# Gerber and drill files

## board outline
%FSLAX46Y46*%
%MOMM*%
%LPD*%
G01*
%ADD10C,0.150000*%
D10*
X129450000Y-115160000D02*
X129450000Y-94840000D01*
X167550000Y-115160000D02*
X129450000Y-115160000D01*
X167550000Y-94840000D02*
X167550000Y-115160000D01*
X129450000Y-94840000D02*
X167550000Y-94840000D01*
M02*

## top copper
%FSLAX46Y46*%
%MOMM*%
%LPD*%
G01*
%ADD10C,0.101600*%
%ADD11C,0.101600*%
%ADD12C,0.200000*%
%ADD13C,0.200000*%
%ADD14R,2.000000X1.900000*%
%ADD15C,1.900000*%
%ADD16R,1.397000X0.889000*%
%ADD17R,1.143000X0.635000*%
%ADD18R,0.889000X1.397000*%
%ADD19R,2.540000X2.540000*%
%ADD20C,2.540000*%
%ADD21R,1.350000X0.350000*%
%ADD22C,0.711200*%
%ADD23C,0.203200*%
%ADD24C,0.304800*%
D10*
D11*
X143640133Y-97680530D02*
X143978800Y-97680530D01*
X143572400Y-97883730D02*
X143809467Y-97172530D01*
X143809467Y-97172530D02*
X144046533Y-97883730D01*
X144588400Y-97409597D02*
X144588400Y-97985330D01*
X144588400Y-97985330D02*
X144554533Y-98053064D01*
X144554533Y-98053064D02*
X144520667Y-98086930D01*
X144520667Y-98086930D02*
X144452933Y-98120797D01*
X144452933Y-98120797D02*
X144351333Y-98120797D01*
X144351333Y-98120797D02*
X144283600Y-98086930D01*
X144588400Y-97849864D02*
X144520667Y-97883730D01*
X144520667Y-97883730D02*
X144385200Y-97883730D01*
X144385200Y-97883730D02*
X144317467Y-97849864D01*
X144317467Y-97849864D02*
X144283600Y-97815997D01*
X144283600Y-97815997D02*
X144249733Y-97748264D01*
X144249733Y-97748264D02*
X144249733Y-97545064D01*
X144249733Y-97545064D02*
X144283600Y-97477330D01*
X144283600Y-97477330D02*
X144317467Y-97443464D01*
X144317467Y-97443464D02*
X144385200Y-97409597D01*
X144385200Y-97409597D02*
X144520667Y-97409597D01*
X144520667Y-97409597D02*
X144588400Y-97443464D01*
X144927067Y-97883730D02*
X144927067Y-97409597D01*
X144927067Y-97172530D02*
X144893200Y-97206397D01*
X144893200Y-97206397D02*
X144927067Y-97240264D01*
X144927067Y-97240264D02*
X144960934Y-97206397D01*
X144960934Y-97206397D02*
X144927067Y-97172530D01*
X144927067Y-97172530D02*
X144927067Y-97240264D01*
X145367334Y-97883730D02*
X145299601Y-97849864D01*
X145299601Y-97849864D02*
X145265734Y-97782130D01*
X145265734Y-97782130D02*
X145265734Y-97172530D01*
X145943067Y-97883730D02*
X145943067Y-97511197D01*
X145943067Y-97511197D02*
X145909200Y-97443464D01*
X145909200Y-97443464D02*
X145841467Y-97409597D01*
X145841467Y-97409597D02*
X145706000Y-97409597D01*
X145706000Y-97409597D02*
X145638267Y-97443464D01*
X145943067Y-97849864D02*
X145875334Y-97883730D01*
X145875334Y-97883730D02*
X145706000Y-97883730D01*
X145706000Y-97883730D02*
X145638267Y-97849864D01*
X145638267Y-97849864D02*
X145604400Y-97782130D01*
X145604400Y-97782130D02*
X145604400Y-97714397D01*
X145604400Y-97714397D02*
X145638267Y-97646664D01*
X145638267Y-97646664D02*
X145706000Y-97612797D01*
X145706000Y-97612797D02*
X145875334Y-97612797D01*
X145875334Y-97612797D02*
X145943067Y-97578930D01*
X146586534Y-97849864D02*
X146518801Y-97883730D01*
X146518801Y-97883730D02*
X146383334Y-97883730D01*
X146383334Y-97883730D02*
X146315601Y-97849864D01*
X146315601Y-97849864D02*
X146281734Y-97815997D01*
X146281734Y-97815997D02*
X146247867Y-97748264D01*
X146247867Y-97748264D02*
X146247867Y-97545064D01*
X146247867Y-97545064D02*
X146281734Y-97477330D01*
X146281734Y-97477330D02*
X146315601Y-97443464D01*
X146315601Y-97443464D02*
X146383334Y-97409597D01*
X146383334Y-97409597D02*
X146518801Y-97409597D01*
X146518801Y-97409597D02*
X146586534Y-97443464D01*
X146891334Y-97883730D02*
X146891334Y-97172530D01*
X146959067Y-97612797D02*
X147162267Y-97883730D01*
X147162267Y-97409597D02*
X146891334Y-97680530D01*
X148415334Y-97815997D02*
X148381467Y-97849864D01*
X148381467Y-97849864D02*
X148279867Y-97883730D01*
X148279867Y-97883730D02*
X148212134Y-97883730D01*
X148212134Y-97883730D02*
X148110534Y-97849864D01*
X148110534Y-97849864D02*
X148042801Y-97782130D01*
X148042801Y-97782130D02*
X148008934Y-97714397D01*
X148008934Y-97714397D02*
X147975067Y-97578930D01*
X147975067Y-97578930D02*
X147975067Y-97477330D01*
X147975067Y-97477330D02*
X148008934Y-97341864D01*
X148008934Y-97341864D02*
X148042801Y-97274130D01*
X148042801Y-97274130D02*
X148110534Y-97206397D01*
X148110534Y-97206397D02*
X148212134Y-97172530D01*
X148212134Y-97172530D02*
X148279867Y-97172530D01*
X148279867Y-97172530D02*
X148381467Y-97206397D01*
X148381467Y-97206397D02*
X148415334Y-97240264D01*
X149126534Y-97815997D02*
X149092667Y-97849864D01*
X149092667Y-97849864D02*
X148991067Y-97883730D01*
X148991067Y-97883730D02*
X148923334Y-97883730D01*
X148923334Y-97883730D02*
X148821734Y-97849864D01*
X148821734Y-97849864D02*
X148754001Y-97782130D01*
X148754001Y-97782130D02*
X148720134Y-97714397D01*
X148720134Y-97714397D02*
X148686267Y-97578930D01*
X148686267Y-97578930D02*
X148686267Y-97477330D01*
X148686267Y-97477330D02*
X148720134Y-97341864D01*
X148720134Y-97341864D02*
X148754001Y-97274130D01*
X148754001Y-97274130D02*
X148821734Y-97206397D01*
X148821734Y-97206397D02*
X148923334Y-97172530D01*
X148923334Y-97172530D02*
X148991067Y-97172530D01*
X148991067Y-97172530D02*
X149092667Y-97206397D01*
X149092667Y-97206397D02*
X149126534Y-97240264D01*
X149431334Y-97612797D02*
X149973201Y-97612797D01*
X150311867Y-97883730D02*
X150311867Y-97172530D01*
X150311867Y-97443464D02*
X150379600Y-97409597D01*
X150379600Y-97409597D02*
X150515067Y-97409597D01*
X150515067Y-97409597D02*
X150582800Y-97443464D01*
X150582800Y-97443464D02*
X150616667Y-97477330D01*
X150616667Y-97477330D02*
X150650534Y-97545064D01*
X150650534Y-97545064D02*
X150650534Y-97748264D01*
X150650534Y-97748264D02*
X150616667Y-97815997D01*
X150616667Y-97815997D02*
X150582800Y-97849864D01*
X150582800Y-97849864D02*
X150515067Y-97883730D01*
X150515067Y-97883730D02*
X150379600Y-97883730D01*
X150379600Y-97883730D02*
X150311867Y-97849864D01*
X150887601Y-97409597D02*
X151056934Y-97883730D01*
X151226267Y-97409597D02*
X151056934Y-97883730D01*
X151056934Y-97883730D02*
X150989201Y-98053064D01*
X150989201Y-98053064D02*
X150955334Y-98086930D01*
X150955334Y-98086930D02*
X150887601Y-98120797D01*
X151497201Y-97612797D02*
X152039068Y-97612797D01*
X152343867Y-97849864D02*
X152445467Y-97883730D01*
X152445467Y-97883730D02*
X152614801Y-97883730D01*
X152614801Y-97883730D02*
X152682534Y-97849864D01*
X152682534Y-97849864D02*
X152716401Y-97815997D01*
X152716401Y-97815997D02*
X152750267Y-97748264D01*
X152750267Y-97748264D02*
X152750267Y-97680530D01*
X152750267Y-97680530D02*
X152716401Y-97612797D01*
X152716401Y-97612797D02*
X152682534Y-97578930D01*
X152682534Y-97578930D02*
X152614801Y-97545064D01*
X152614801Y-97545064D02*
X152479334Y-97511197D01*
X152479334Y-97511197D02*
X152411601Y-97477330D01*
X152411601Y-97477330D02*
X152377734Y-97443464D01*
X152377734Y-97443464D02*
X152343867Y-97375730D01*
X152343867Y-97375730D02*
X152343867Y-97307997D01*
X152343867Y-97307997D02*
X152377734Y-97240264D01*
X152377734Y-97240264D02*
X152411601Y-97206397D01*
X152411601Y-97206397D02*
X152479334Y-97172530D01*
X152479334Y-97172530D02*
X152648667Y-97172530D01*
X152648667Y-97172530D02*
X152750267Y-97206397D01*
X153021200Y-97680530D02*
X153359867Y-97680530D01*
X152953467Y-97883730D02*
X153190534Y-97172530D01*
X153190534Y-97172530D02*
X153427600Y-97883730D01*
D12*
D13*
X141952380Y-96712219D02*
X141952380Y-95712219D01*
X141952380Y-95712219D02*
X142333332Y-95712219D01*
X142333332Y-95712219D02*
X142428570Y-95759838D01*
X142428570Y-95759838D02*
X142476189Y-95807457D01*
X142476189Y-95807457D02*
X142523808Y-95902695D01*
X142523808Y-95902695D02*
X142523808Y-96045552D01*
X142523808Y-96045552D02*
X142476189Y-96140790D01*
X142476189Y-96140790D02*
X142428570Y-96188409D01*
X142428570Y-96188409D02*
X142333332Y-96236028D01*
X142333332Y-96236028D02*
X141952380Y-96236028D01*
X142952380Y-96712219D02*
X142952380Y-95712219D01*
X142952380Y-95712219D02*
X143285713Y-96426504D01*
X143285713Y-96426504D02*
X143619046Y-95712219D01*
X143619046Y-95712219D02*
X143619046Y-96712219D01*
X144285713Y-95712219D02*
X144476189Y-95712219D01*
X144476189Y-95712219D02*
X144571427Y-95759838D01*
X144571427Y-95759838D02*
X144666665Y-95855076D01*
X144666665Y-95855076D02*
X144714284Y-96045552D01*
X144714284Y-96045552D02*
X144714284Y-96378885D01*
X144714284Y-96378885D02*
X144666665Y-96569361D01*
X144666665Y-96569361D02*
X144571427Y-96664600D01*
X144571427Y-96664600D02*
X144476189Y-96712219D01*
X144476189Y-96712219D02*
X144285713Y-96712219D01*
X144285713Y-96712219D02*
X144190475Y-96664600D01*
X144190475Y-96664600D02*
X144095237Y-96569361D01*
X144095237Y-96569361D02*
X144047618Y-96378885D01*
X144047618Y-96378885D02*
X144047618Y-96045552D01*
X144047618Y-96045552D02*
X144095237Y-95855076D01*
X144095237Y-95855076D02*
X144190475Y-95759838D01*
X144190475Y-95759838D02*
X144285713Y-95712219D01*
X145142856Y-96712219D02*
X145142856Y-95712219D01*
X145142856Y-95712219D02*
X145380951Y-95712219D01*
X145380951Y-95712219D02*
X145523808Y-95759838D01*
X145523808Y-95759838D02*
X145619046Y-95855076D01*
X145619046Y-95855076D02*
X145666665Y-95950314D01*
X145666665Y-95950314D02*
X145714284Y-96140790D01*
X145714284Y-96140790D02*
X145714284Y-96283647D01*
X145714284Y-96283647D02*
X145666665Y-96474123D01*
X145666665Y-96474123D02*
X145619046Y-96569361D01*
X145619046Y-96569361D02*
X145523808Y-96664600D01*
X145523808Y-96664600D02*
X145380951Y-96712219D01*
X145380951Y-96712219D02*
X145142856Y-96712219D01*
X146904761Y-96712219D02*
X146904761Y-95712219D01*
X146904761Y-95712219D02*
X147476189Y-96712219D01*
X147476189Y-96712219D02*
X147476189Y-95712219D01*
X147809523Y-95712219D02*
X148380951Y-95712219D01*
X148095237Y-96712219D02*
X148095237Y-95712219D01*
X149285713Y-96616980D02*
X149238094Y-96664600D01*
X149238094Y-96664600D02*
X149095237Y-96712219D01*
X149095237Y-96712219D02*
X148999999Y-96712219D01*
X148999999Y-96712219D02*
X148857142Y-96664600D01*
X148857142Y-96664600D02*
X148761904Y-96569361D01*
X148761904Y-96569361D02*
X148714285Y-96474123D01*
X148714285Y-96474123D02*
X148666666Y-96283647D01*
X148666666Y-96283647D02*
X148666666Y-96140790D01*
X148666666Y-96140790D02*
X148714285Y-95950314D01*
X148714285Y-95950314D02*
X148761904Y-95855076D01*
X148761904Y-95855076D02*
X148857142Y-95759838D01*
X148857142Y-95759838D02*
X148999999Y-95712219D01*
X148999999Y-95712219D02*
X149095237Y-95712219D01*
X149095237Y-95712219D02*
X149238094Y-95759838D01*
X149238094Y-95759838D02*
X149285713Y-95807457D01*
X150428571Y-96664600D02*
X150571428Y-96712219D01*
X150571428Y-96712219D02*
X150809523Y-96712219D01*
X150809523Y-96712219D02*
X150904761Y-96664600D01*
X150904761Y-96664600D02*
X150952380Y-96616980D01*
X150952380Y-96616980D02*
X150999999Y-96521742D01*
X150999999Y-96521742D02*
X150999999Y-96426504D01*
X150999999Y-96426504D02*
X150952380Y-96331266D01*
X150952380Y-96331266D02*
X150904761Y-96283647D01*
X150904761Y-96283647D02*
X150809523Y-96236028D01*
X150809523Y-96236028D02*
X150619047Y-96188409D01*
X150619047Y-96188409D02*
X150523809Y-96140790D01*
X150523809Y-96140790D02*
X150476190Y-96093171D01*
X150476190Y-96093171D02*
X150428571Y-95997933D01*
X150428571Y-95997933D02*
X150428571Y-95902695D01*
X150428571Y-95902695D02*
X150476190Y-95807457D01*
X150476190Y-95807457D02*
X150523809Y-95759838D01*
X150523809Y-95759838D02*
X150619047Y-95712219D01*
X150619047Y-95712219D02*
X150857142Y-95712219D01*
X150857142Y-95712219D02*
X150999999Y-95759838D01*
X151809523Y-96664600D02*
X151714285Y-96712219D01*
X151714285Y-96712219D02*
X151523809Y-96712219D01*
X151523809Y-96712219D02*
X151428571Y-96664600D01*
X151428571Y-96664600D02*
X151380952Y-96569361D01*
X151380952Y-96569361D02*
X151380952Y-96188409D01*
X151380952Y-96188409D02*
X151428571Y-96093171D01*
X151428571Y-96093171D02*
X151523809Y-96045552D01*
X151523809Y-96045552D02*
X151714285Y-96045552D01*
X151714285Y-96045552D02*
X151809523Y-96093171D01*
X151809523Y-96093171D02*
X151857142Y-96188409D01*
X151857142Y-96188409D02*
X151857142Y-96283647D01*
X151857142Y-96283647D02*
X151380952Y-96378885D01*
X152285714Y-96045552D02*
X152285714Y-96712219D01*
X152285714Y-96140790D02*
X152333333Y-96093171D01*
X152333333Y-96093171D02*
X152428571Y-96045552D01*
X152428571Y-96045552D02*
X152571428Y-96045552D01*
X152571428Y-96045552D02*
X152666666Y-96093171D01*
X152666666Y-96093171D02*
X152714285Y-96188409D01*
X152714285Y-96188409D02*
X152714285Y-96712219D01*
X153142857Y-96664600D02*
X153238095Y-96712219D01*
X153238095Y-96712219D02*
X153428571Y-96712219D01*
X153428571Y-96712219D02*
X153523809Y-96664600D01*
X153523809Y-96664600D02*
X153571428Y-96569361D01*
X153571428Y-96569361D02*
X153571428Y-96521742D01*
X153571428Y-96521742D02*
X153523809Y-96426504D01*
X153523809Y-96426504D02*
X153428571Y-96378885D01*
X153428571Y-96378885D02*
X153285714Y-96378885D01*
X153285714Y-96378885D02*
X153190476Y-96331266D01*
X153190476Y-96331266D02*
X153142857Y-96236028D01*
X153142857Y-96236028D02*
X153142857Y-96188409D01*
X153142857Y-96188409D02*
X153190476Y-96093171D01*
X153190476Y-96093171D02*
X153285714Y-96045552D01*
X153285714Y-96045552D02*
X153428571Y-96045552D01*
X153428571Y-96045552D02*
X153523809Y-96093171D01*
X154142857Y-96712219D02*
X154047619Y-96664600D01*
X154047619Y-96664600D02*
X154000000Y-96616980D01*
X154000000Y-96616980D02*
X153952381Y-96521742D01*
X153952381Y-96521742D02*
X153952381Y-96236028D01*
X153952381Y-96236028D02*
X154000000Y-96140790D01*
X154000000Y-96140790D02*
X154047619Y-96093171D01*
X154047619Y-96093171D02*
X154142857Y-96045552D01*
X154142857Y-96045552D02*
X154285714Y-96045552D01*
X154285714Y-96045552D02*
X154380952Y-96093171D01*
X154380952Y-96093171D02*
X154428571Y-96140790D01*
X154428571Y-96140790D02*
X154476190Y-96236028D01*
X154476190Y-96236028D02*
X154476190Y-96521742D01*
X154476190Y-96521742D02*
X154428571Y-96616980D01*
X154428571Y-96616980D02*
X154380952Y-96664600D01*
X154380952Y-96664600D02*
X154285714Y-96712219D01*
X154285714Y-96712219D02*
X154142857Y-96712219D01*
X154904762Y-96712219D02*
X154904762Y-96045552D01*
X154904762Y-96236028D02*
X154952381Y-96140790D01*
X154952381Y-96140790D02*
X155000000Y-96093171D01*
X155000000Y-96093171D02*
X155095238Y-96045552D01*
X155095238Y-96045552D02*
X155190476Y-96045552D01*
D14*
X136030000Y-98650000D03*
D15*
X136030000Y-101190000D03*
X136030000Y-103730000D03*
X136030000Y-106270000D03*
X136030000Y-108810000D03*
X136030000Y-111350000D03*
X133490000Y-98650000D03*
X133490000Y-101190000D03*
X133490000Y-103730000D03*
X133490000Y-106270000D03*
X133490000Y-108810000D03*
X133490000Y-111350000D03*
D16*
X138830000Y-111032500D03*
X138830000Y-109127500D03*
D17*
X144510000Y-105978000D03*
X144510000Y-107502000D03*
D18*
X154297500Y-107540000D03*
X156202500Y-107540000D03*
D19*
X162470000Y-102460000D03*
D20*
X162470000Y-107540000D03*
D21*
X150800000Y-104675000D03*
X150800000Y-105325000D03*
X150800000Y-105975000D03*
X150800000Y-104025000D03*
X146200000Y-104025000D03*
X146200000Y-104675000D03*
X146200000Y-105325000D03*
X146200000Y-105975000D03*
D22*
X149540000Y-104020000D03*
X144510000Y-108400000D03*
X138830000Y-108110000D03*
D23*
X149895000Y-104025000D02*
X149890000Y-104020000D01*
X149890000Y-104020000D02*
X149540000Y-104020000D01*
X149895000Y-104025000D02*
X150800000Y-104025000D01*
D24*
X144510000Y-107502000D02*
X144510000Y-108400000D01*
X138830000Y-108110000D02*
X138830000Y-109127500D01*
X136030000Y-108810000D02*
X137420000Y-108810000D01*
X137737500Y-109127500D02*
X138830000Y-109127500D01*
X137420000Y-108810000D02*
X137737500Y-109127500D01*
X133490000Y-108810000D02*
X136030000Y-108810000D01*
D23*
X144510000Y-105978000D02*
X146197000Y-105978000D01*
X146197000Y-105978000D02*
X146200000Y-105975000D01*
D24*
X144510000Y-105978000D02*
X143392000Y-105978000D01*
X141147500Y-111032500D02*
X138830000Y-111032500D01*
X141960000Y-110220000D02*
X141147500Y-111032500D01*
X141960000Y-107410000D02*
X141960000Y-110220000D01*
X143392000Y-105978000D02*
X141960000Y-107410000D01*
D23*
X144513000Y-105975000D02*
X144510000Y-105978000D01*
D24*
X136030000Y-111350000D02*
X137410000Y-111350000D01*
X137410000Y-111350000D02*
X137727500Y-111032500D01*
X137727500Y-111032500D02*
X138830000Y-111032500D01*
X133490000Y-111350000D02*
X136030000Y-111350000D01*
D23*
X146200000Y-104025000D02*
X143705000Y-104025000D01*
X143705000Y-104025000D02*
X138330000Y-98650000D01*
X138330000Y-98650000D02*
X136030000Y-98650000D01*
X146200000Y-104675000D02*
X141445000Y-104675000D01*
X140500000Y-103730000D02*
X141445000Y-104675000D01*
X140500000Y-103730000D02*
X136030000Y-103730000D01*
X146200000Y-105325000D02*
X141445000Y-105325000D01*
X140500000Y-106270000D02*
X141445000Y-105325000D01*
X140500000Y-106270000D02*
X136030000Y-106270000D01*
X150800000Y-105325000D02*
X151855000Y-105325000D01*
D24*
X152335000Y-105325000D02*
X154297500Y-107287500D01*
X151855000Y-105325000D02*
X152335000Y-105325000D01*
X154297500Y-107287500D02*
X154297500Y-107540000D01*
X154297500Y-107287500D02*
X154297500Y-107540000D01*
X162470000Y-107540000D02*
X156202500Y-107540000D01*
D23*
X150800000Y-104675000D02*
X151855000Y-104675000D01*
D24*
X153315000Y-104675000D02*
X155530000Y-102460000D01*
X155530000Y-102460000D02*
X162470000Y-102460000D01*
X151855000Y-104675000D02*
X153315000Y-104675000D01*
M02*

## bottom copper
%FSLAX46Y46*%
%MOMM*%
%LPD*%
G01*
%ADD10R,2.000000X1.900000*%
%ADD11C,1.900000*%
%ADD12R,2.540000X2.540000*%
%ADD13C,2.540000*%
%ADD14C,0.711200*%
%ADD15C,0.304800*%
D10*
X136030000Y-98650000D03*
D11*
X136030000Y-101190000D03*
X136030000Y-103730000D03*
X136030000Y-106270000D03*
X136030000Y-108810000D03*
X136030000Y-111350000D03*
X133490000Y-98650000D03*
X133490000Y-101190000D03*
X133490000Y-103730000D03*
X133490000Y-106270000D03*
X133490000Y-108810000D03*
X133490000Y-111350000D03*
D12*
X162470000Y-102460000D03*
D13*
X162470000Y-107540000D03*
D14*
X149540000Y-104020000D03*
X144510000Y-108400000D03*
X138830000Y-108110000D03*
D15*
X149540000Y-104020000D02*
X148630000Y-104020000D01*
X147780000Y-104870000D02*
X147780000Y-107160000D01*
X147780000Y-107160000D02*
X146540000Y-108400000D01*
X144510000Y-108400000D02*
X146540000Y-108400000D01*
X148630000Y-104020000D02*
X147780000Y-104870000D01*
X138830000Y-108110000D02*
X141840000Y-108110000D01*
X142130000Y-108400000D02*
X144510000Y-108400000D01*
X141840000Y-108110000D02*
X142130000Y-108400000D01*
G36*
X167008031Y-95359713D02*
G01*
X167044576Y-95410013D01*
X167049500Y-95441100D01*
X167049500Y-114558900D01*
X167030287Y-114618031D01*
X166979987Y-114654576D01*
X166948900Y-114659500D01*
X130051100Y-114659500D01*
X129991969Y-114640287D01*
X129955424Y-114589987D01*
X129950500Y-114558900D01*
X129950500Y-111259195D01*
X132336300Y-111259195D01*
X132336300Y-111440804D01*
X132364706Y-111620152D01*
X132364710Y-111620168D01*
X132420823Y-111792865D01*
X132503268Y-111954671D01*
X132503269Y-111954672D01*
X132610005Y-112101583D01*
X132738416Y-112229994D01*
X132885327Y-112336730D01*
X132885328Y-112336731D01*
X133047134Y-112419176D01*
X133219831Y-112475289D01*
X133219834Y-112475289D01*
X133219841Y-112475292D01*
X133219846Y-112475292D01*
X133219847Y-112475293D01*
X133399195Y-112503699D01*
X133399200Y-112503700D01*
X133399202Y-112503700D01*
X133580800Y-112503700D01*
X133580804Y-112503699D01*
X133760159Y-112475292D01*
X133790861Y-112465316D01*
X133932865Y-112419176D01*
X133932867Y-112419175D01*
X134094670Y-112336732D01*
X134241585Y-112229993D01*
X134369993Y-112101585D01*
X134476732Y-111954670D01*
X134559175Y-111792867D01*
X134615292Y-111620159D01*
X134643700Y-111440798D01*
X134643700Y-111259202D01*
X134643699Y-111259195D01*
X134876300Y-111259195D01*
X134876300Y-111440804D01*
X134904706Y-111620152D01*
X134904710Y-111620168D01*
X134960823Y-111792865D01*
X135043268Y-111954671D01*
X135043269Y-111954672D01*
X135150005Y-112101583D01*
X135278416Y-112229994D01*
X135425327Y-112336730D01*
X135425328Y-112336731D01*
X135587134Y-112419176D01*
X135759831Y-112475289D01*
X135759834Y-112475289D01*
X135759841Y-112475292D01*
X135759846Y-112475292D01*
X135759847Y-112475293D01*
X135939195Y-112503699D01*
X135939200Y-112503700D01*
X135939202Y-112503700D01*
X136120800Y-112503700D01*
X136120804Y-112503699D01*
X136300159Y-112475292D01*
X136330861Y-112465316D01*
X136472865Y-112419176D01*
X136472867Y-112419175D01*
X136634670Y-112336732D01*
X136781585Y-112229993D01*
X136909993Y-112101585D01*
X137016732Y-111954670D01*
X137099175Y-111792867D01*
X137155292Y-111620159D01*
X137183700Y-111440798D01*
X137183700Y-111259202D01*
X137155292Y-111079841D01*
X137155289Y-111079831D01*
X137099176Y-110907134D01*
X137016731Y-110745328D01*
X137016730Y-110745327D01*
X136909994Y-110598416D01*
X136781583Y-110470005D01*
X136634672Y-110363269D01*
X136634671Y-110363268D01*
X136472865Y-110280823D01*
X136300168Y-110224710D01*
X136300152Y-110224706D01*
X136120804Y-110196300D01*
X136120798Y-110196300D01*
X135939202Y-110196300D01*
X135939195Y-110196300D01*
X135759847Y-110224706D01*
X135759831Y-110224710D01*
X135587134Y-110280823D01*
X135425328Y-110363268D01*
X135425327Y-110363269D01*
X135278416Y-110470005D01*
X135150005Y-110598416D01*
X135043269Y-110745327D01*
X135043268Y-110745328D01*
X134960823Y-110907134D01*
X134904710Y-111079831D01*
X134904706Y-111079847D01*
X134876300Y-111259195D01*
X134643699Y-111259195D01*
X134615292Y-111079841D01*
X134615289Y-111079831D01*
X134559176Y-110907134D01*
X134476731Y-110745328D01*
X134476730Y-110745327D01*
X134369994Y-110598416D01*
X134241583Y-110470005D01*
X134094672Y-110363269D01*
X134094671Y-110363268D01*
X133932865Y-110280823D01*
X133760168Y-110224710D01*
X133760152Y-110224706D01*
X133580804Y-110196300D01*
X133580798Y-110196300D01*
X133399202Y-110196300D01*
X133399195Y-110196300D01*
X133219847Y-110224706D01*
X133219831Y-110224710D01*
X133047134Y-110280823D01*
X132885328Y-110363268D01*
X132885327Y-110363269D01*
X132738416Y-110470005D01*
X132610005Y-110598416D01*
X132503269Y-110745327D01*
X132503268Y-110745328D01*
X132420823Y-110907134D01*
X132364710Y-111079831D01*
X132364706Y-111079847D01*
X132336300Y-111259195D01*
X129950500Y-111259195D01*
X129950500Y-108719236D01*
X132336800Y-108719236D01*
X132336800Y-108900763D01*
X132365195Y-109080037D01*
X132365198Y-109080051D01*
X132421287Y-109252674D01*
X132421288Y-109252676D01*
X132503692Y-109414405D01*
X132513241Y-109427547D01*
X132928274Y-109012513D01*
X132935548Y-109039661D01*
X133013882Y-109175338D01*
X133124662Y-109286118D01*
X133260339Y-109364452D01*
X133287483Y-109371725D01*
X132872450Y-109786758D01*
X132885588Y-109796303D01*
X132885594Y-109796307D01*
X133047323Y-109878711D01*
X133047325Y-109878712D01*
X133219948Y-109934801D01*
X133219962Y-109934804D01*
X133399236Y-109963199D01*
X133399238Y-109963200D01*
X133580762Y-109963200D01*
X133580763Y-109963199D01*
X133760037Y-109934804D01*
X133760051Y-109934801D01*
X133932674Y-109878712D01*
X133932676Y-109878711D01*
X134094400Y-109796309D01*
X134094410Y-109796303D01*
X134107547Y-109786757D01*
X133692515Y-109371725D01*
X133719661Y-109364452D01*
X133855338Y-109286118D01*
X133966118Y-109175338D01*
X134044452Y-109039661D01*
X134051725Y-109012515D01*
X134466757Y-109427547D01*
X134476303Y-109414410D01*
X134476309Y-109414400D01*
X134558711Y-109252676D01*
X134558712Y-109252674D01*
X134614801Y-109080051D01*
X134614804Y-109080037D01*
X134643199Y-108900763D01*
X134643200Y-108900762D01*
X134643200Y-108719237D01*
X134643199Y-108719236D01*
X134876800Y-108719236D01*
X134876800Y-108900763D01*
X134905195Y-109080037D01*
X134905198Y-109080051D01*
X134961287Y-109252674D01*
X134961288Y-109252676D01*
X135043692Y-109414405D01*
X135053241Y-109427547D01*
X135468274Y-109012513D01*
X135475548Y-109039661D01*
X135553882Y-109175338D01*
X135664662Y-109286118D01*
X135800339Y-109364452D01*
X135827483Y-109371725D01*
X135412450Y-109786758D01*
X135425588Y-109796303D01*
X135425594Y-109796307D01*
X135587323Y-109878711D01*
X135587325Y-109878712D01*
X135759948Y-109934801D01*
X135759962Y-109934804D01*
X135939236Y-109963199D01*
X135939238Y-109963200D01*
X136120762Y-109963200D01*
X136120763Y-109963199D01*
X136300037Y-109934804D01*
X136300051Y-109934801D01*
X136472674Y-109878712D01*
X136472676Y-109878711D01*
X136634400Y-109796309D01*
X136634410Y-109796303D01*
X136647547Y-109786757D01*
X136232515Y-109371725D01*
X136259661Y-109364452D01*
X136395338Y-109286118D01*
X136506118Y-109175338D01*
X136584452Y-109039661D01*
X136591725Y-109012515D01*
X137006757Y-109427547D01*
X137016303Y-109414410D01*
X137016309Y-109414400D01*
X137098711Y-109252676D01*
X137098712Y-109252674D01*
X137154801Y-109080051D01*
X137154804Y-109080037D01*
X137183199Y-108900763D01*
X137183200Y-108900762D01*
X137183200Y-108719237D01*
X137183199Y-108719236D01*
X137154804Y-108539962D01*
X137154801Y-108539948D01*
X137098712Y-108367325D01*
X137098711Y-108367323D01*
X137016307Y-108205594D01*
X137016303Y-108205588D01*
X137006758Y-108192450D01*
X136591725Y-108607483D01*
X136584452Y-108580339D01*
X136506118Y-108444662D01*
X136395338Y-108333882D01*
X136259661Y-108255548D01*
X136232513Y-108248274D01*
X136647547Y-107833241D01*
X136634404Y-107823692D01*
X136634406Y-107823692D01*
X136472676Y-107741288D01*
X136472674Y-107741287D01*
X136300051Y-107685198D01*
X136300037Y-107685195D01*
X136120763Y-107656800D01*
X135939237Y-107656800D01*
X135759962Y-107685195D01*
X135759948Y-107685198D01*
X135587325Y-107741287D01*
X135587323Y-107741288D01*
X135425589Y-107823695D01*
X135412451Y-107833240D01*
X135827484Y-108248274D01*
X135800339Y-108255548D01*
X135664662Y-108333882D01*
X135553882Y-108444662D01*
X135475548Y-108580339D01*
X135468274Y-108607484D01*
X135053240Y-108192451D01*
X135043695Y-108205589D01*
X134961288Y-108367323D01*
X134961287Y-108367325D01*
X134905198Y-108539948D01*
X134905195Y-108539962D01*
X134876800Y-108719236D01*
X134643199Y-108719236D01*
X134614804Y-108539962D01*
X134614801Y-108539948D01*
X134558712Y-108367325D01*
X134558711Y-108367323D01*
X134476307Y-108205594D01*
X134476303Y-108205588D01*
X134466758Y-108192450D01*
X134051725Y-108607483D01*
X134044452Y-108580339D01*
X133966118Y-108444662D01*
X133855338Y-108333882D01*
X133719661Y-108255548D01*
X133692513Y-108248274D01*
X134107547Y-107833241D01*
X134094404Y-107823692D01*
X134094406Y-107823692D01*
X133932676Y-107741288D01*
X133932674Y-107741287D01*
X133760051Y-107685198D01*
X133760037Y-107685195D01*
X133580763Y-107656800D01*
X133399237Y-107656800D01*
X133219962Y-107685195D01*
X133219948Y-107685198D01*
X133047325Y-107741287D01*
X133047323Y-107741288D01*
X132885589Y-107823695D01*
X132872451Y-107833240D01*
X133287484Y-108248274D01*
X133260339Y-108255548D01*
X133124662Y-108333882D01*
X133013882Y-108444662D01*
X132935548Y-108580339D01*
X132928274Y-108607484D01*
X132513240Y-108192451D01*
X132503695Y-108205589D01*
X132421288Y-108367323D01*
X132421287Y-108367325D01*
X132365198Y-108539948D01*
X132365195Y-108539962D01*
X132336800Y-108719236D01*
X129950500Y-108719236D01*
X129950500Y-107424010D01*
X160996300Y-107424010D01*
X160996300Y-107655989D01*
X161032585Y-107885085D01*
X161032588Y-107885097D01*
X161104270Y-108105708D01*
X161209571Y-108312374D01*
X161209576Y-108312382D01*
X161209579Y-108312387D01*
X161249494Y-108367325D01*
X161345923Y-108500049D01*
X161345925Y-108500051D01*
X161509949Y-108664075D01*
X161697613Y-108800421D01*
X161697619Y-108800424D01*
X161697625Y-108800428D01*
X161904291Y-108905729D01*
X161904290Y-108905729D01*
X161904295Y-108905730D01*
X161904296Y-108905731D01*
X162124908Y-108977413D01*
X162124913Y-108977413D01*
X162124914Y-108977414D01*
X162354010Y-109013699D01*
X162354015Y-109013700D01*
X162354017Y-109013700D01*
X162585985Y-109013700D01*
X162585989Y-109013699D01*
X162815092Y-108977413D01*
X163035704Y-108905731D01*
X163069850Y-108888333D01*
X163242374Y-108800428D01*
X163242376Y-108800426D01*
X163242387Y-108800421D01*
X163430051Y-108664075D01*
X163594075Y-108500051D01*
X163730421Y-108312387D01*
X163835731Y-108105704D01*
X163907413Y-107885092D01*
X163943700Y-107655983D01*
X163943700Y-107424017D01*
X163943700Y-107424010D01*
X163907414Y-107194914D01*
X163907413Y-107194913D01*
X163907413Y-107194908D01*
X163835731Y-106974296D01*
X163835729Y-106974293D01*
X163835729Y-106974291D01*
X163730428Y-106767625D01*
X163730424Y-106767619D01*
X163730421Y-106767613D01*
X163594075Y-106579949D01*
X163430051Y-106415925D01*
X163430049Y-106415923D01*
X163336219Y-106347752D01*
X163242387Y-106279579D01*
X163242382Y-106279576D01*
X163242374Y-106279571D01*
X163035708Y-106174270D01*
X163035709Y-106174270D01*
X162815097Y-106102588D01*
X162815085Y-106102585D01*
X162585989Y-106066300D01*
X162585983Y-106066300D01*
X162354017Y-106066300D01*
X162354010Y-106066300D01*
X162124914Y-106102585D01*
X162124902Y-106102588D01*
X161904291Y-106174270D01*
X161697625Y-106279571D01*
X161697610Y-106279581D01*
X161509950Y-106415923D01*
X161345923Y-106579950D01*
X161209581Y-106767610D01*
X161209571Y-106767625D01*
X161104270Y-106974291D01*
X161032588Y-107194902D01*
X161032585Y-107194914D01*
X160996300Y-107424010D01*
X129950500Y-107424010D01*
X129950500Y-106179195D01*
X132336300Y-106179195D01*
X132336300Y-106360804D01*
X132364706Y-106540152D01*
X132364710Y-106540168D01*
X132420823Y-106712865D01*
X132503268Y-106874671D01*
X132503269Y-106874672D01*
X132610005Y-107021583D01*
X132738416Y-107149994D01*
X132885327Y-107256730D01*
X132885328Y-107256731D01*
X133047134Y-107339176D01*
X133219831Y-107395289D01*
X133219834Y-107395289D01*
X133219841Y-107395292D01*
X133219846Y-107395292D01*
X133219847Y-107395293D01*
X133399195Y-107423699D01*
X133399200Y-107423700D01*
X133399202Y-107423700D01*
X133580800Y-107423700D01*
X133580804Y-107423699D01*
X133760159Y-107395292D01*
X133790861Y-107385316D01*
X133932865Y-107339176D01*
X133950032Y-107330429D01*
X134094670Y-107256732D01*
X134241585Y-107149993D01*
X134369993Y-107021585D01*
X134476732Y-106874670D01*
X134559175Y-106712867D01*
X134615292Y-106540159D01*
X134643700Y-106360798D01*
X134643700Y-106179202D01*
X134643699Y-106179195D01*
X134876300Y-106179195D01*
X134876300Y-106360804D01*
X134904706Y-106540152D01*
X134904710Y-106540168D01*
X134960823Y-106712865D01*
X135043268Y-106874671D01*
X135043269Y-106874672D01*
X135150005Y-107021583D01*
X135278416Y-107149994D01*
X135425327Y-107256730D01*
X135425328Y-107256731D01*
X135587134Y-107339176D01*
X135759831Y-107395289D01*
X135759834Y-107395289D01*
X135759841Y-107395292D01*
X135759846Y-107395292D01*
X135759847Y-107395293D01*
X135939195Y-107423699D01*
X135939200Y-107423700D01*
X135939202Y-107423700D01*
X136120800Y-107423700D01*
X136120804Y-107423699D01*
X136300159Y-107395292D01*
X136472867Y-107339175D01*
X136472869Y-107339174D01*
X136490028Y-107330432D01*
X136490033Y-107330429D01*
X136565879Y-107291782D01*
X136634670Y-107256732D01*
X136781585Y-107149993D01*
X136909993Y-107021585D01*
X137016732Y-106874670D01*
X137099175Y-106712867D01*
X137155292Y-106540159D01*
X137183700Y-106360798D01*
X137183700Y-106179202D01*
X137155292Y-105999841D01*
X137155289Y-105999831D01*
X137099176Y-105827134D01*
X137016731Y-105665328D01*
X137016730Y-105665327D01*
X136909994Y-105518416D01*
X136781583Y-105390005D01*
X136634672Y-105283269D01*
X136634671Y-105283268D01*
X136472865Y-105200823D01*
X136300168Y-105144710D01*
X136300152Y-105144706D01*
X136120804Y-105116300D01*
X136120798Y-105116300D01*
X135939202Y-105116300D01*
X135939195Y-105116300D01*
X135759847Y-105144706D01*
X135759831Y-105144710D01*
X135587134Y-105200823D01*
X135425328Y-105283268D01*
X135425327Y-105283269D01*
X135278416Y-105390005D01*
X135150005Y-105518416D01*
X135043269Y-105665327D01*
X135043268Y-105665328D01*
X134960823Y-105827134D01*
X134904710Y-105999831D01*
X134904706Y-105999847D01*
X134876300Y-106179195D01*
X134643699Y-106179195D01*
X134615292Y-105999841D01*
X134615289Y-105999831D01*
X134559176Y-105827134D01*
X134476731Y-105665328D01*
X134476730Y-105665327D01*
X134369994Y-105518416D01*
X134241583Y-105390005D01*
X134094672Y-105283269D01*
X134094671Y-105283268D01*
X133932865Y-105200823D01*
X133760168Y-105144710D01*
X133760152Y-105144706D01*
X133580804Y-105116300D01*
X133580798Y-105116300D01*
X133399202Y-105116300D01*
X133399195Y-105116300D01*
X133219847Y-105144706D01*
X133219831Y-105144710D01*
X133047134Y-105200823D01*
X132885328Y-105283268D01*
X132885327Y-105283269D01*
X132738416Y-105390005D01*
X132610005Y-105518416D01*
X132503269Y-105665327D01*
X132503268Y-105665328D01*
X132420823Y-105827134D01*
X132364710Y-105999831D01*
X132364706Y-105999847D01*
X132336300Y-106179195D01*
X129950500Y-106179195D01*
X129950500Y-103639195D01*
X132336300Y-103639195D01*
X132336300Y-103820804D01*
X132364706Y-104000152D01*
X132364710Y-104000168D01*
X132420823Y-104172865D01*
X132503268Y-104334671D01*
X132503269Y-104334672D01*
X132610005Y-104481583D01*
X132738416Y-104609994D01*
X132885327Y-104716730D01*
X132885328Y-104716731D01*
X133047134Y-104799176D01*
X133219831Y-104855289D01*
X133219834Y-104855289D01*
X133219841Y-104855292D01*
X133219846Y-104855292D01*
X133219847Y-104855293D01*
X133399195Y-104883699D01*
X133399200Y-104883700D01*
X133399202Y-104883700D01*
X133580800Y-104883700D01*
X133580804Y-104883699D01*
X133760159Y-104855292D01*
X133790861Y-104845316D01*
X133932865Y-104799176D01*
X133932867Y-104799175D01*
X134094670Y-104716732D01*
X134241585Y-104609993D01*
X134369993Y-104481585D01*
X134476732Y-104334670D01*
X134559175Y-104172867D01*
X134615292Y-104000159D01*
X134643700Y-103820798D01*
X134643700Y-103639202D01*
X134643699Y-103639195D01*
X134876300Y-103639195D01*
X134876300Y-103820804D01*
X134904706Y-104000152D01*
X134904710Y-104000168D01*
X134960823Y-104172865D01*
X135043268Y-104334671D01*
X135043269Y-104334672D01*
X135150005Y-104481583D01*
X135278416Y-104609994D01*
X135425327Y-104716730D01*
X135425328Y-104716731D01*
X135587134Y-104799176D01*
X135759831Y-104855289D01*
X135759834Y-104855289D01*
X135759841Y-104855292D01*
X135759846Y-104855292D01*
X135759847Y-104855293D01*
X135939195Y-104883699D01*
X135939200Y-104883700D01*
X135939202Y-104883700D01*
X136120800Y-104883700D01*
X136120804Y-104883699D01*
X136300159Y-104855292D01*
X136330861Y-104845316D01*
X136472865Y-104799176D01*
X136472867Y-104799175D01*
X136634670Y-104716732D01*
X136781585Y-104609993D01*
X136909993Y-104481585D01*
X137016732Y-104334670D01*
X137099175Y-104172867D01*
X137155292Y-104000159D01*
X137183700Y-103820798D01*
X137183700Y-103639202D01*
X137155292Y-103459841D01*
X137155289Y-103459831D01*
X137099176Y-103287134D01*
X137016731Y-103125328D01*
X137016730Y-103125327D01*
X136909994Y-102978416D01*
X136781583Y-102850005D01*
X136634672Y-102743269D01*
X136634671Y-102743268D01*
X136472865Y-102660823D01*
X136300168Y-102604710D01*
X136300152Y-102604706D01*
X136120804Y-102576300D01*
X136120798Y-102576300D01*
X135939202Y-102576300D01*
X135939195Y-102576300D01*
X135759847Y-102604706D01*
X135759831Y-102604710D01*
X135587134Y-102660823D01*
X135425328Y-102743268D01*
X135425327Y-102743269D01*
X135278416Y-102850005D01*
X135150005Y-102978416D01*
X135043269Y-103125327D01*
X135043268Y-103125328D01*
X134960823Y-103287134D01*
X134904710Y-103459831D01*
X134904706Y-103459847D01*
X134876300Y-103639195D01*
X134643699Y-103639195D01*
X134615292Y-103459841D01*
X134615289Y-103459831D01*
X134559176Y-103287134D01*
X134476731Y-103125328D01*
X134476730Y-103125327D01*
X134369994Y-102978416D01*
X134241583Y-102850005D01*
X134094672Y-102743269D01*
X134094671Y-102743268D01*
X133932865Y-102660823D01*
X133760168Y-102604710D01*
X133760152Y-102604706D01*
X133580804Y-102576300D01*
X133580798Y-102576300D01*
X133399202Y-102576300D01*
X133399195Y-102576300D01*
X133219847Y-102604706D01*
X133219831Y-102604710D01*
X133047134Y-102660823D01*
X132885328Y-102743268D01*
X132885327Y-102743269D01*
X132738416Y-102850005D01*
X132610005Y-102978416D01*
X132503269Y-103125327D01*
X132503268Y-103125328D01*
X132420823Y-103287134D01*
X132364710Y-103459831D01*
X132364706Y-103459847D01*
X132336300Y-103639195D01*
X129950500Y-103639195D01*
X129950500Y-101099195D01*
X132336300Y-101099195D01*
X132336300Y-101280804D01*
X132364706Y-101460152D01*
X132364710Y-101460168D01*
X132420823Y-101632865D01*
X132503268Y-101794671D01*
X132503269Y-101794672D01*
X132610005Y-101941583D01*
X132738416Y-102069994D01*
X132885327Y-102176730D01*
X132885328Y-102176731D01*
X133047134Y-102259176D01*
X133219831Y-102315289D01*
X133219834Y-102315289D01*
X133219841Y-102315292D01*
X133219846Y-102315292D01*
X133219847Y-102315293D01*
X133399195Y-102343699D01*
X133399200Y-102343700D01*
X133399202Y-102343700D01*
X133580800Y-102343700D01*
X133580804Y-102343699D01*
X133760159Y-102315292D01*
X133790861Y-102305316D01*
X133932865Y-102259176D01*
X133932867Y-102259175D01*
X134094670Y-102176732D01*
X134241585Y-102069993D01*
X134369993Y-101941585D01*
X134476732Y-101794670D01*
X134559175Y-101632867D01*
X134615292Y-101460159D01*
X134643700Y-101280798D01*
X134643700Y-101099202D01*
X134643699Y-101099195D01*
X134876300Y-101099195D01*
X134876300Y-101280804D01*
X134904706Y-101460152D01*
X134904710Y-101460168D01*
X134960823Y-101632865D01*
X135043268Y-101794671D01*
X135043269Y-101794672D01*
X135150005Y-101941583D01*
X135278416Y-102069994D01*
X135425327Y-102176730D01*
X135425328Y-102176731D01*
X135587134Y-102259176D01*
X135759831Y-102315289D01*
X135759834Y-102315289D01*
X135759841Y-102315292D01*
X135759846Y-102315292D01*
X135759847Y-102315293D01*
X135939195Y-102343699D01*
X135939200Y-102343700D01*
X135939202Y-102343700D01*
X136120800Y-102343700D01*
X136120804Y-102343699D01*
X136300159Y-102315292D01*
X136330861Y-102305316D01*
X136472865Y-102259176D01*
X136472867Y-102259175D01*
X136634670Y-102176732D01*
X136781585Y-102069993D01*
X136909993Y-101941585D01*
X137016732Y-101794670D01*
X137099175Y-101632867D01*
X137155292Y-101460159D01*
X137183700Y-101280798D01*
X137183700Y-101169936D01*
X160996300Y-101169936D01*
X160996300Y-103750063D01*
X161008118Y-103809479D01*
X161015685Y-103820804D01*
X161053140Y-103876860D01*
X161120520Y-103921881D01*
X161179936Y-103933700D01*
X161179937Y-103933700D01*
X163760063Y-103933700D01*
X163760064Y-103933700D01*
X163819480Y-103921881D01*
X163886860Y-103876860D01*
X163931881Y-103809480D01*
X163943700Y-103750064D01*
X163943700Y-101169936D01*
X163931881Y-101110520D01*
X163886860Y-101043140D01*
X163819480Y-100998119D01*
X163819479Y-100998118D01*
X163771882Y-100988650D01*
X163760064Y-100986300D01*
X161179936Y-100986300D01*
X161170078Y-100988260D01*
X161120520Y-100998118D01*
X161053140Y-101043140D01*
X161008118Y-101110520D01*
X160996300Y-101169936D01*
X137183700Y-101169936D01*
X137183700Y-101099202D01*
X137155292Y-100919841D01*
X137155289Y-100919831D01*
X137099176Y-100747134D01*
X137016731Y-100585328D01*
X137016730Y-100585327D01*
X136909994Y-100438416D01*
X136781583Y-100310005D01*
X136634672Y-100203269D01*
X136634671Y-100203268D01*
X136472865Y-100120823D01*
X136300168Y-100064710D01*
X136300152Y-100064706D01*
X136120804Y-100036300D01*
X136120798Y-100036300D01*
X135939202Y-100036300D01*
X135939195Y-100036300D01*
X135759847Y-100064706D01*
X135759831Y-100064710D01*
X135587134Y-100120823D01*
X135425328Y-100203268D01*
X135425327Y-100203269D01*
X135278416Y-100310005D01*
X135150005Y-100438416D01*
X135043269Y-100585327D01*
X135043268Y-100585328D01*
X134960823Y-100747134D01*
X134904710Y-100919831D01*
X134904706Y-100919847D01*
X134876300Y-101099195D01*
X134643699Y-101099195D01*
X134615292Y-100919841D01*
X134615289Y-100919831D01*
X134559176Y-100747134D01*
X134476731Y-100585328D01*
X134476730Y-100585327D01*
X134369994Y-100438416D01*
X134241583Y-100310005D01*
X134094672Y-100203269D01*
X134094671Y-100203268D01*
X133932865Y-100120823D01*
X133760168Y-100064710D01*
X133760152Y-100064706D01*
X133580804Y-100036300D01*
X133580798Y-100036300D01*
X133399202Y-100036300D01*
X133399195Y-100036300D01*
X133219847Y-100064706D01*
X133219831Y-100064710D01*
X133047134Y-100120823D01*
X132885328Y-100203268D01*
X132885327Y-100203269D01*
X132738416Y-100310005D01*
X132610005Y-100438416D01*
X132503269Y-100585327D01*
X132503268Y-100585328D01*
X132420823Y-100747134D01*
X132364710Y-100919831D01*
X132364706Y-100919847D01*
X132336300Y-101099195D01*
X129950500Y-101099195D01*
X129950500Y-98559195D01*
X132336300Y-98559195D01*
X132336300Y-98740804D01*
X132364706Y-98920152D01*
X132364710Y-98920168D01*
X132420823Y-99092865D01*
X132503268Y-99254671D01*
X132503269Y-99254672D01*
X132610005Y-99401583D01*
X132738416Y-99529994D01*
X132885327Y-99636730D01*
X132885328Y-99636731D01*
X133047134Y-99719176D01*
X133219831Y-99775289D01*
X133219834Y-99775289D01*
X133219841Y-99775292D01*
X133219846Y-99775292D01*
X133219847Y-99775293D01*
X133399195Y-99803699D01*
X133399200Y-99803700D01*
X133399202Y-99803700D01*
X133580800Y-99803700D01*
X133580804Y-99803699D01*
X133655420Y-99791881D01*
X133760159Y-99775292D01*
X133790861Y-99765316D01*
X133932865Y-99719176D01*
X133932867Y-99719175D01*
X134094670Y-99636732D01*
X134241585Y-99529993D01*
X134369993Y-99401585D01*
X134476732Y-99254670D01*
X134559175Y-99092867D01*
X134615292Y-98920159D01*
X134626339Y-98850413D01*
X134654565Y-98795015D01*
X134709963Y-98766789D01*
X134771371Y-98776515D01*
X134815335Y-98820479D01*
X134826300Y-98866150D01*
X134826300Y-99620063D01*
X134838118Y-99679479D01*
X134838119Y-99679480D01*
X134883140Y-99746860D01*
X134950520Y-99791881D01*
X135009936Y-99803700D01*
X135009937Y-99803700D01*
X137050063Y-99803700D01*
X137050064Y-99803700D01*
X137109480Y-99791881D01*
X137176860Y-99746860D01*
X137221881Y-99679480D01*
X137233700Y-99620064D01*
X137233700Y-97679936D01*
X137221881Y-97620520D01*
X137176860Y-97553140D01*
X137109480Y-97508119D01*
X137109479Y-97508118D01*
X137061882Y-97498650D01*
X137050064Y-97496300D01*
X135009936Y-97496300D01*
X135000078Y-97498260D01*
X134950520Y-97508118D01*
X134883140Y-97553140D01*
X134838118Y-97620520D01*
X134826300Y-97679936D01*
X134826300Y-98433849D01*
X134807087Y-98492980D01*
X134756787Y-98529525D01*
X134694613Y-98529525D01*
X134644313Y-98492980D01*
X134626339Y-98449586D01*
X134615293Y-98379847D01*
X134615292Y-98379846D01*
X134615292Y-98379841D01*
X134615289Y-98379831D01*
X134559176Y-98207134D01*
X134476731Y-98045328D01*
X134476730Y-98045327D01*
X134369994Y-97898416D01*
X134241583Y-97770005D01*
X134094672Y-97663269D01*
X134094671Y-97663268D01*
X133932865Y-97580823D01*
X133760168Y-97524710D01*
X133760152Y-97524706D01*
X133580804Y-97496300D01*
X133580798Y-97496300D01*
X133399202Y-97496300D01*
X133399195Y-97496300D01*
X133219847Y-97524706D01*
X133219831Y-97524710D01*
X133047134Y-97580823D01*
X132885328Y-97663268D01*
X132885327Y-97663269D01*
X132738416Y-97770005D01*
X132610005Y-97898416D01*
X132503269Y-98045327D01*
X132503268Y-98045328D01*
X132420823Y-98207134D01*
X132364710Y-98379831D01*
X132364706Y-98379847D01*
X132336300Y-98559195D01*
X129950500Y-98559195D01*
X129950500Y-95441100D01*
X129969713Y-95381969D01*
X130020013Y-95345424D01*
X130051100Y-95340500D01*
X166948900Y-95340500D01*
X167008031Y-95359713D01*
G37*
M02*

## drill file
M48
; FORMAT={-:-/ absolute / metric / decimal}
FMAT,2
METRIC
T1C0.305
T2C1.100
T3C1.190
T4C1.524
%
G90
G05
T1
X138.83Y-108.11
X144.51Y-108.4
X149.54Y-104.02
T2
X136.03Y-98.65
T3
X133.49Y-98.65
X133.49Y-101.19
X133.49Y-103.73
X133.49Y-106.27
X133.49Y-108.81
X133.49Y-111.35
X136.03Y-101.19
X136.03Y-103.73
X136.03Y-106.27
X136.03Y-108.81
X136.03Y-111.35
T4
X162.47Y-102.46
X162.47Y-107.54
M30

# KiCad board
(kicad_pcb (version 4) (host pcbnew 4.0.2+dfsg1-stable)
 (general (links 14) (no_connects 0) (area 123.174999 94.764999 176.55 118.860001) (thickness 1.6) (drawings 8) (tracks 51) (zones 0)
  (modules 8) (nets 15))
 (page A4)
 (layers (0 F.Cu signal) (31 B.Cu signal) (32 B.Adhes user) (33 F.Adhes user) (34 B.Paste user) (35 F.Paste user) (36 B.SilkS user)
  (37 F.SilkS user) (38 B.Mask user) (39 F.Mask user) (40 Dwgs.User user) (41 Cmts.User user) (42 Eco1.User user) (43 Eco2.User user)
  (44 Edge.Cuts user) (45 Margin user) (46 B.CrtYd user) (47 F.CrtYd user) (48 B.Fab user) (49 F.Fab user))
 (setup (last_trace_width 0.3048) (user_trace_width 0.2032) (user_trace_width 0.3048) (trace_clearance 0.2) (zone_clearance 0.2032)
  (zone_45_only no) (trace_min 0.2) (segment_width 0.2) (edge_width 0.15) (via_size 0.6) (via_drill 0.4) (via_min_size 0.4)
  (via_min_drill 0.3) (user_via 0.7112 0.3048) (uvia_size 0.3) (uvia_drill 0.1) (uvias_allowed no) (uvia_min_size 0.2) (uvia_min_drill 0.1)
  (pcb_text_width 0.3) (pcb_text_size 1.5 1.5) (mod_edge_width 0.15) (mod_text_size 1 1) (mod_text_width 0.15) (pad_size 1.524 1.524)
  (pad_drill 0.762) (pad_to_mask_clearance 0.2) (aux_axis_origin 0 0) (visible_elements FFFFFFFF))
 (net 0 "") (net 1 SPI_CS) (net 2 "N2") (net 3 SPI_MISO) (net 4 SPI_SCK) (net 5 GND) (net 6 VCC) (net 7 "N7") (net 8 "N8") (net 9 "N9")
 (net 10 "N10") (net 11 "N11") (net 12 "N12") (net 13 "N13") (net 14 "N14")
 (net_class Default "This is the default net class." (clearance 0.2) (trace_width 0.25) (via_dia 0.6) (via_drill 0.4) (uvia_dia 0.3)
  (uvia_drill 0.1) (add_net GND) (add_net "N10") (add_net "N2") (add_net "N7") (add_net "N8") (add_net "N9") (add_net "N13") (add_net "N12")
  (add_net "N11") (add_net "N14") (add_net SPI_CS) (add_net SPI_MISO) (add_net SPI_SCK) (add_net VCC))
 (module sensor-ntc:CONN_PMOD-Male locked (layer F.Cu) (at 133.49 105 90)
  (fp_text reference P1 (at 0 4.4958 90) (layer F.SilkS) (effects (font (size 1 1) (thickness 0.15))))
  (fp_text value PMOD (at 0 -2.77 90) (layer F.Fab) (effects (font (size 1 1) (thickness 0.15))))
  (pad 1 thru_hole rect (at 6.35 2.54 90) (size 1.9 2) (drill 1.1) (layers *.Cu *.Mask) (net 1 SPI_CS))
  (pad 2 thru_hole circle (at 3.81 2.54 90) (size 1.9 1.9) (drill 1.19) (layers *.Cu *.Mask) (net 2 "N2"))
  (pad 3 thru_hole circle (at 1.27 2.54 90) (size 1.9 1.9) (drill 1.19) (layers *.Cu *.Mask) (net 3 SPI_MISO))
  (pad 4 thru_hole circle (at -1.27 2.54 90) (size 1.9 1.9) (drill 1.19) (layers *.Cu *.Mask) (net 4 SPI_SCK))
  (pad 5 thru_hole circle (at -3.81 2.54 90) (size 1.9 1.9) (drill 1.19) (layers *.Cu *.Mask) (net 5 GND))
  (pad 6 thru_hole circle (at -6.35 2.54 90) (size 1.9 1.9) (drill 1.19) (layers *.Cu *.Mask) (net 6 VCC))
  (pad 7 thru_hole circle (at 6.35 0 90) (size 1.9 1.9) (drill 1.19) (layers *.Cu *.Mask) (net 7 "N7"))
  (pad 8 thru_hole circle (at 3.81 0 90) (size 1.9 1.9) (drill 1.19) (layers *.Cu *.Mask) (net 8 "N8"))
  (pad 9 thru_hole circle (at 1.27 0 90) (size 1.9 1.9) (drill 1.19) (layers *.Cu *.Mask) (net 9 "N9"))
  (pad 10 thru_hole circle (at -1.27 0 90) (size 1.9 1.9) (drill 1.19) (layers *.Cu *.Mask) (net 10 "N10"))
  (pad 11 thru_hole circle (at -3.81 0 90) (size 1.9 1.9) (drill 1.19) (layers *.Cu *.Mask) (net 5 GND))
  (pad 12 thru_hole circle (at -6.35 0 90) (size 1.9 1.9) (drill 1.19) (layers *.Cu *.Mask) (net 6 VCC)))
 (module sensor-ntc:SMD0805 (layer F.Cu) (at 138.83 110.08 90)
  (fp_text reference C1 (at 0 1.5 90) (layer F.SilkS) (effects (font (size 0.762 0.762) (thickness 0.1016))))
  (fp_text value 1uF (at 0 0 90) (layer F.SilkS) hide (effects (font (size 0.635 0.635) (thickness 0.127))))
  (pad 1 smd rect (at -0.9525 0 90) (size 0.889 1.397) (layers F.Cu F.Paste F.Mask) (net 6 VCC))
  (pad 2 smd rect (at 0.9525 0 90) (size 0.889 1.397) (layers F.Cu F.Paste F.Mask) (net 5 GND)))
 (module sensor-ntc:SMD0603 (layer F.Cu) (at 144.51 106.74 270)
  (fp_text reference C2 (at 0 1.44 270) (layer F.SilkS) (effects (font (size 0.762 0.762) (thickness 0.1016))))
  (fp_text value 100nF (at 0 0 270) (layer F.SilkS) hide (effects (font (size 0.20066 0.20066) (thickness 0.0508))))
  (pad 1 smd rect (at -0.762 0 270) (size 0.635 1.143) (layers F.Cu F.Paste F.Mask) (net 6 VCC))
  (pad 2 smd rect (at 0.762 0 270) (size 0.635 1.143) (layers F.Cu F.Paste F.Mask) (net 5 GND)))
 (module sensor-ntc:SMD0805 (layer F.Cu) (at 155.25 107.54)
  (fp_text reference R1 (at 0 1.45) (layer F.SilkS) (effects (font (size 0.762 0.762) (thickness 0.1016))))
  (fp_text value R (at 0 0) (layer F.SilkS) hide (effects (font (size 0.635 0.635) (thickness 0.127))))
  (pad 1 smd rect (at -0.9525 0) (size 0.889 1.397) (layers F.Cu F.Paste F.Mask) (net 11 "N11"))
  (pad 2 smd rect (at 0.9525 0) (size 0.889 1.397) (layers F.Cu F.Paste F.Mask) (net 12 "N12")))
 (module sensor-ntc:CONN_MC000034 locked (layer F.Cu) (at 162.47 105 270)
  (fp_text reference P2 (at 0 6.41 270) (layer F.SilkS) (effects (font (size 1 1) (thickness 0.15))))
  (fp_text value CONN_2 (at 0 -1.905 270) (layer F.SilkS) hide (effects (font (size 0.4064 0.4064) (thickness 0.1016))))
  (pad 1 thru_hole rect (at -2.54 0 270) (size 2.54 2.54) (drill 1.524) (layers *.Cu *.Mask F.SilkS) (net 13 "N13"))
  (pad 2 thru_hole circle (at 2.54 0 270) (size 2.54 2.54) (drill 1.524) (layers *.Cu *.Mask F.SilkS) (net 12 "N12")))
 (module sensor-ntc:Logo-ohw (layer F.Cu) (at 148.5 110)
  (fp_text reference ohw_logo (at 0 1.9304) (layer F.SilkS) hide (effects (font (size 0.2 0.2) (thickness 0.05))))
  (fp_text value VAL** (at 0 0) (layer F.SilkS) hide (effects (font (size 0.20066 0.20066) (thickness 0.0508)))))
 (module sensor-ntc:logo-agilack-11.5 (layer F.Cu) (at 161.56 112.74)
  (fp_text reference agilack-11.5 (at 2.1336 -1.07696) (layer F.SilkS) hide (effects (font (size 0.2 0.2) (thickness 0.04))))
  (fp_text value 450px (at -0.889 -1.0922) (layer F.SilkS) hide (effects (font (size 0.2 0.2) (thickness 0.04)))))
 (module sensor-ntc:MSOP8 (layer F.Cu) (at 148.5 105 90)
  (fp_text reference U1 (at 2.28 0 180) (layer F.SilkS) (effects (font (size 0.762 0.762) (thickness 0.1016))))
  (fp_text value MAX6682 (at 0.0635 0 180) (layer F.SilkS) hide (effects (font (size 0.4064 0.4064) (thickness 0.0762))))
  (pad 3 smd rect (at 0.325 2.3 90) (size 0.35 1.35) (layers F.Cu F.Paste F.Mask) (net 13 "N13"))
  (pad 2 smd rect (at -0.325 2.3 90) (size 0.35 1.35) (layers F.Cu F.Paste F.Mask) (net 11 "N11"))
  (pad 1 smd rect (at -0.975 2.3 90) (size 0.35 1.35) (layers F.Cu F.Paste F.Mask) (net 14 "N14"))
  (pad 4 smd rect (at 0.975 2.3 90) (size 0.35 1.35) (layers F.Cu F.Paste F.Mask) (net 5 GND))
  (pad 5 smd rect (at 0.975 -2.3 90) (size 0.35 1.35) (layers F.Cu F.Paste F.Mask) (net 1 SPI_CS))
  (pad 6 smd rect (at 0.325 -2.3 90) (size 0.35 1.35) (layers F.Cu F.Paste F.Mask) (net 3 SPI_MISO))
  (pad 7 smd rect (at -0.325 -2.3 90) (size 0.35 1.35) (layers F.Cu F.Paste F.Mask) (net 4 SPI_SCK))
  (pad 8 smd rect (at -0.975 -2.3 90) (size 0.35 1.35) (layers F.Cu F.Paste F.Mask) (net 6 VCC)))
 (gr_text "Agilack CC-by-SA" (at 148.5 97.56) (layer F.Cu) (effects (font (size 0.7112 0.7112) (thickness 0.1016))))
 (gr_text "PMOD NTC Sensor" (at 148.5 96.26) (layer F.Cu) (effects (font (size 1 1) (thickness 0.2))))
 (gr_line (start 129.45 115.16) (end 129.45 94.84) (angle 90) (layer Edge.Cuts) (width 0.15))
 (gr_line (start 167.55 115.16) (end 129.45 115.16) (angle 90) (layer Edge.Cuts) (width 0.15))
 (gr_line (start 167.55 94.84) (end 167.55 115.16) (angle 90) (layer Edge.Cuts) (width 0.15))
 (gr_line (start 129.45 94.84) (end 167.55 94.84) (angle 90) (layer Edge.Cuts) (width 0.15))
 (segment (start 149.54 104.02) (end 148.63 104.02) (width 0.3048) (layer B.Cu) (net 5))
 (segment (start 147.78 104.87) (end 147.78 107.16) (width 0.3048) (layer B.Cu) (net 5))
 (segment (start 147.78 107.16) (end 146.54 108.4) (width 0.3048) (layer B.Cu) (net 5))
 (segment (start 144.51 108.4) (end 146.54 108.4) (width 0.3048) (layer B.Cu) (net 5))
 (segment (start 149.895 104.025) (end 149.89 104.02) (width 0.2032) (layer F.Cu) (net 5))
 (segment (start 149.89 104.02) (end 149.54 104.02) (width 0.2032) (layer F.Cu) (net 5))
 (via (at 149.54 104.02) (size 0.7112) (drill 0.3048) (layers F.Cu B.Cu) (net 5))
 (segment (start 149.895 104.025) (end 150.8 104.025) (width 0.2032) (layer F.Cu) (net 5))
 (segment (start 148.63 104.02) (end 147.78 104.87) (width 0.3048) (layer B.Cu) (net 5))
 (segment (start 138.83 108.11) (end 141.84 108.11) (width 0.3048) (layer B.Cu) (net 5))
 (via (at 144.51 108.4) (size 0.7112) (drill 0.3048) (layers F.Cu B.Cu) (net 5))
 (segment (start 144.51 107.502) (end 144.51 108.4) (width 0.3048) (layer F.Cu) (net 5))
 (via (at 138.83 108.11) (size 0.7112) (drill 0.3048) (layers F.Cu B.Cu) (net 5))
 (segment (start 138.83 108.11) (end 138.83 109.1275) (width 0.3048) (layer F.Cu) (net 5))
 (segment (start 142.13 108.4) (end 144.51 108.4) (width 0.3048) (layer B.Cu) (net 5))
 (segment (start 141.84 108.11) (end 142.13 108.4) (width 0.3048) (layer B.Cu) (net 5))
 (segment (start 136.03 108.81) (end 137.42 108.81) (width 0.3048) (layer F.Cu) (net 5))
 (segment (start 137.7375 109.1275) (end 138.83 109.1275) (width 0.3048) (layer F.Cu) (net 5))
 (segment (start 137.42 108.81) (end 137.7375 109.1275) (width 0.3048) (layer F.Cu) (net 5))
 (segment (start 133.49 108.81) (end 136.03 108.81) (width 0.3048) (layer F.Cu) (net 5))
 (segment (start 144.51 105.978) (end 146.197 105.978) (width 0.2032) (layer F.Cu) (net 6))
 (segment (start 146.197 105.978) (end 146.2 105.975) (width 0.2032) (layer F.Cu) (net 6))
 (segment (start 144.51 105.978) (end 143.392 105.978) (width 0.3048) (layer F.Cu) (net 6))
 (segment (start 141.1475 111.0325) (end 138.83 111.0325) (width 0.3048) (layer F.Cu) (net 6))
 (segment (start 141.96 110.22) (end 141.1475 111.0325) (width 0.3048) (layer F.Cu) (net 6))
 (segment (start 141.96 107.41) (end 141.96 110.22) (width 0.3048) (layer F.Cu) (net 6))
 (segment (start 143.392 105.978) (end 141.96 107.41) (width 0.3048) (layer F.Cu) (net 6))
 (segment (start 144.513 105.975) (end 144.51 105.978) (width 0.2032) (layer F.Cu) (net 6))
 (segment (start 136.03 111.35) (end 137.41 111.35) (width 0.3048) (layer F.Cu) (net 6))
 (segment (start 137.41 111.35) (end 137.7275 111.0325) (width 0.3048) (layer F.Cu) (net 6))
 (segment (start 137.7275 111.0325) (end 138.83 111.0325) (width 0.3048) (layer F.Cu) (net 6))
 (segment (start 133.49 111.35) (end 136.03 111.35) (width 0.3048) (layer F.Cu) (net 6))
 (segment (start 146.2 104.025) (end 143.705 104.025) (width 0.2032) (layer F.Cu) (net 1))
 (segment (start 143.705 104.025) (end 138.33 98.65) (width 0.2032) (layer F.Cu) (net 1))
 (segment (start 138.33 98.65) (end 136.03 98.65) (width 0.2032) (layer F.Cu) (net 1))
 (segment (start 146.2 104.675) (end 141.445 104.675) (width 0.2032) (layer F.Cu) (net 3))
 (segment (start 140.5 103.73) (end 141.445 104.675) (width 0.2032) (layer F.Cu) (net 3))
 (segment (start 140.5 103.73) (end 136.03 103.73) (width 0.2032) (layer F.Cu) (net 3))
 (segment (start 146.2 105.325) (end 141.445 105.325) (width 0.2032) (layer F.Cu) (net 4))
 (segment (start 140.5 106.27) (end 141.445 105.325) (width 0.2032) (layer F.Cu) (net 4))
 (segment (start 140.5 106.27) (end 136.03 106.27) (width 0.2032) (layer F.Cu) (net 4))
 (segment (start 150.8 105.325) (end 151.855 105.325) (width 0.2032) (layer F.Cu) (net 11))
 (segment (start 152.335 105.325) (end 154.2975 107.2875) (width 0.3048) (layer F.Cu) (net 11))
 (segment (start 151.855 105.325) (end 152.335 105.325) (width 0.3048) (layer F.Cu) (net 11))
 (segment (start 154.2975 107.2875) (end 154.2975 107.54) (width 0.3048) (layer F.Cu) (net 11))
 (segment (start 154.2975 107.2875) (end 154.2975 107.54) (width 0.3048) (layer F.Cu) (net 11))
 (segment (start 162.47 107.54) (end 156.2025 107.54) (width 0.3048) (layer F.Cu) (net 12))
 (segment (start 150.8 104.675) (end 151.855 104.675) (width 0.2032) (layer F.Cu) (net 13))
 (segment (start 153.315 104.675) (end 155.53 102.46) (width 0.3048) (layer F.Cu) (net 13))
 (segment (start 155.53 102.46) (end 162.47 102.46) (width 0.3048) (layer F.Cu) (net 13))
 (segment (start 151.855 104.675) (end 153.315 104.675) (width 0.3048) (layer F.Cu) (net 13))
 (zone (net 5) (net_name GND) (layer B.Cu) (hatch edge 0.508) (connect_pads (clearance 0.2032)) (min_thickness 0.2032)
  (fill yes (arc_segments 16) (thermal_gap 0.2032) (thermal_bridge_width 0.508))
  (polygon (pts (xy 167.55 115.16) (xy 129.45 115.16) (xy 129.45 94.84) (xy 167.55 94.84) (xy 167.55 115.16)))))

